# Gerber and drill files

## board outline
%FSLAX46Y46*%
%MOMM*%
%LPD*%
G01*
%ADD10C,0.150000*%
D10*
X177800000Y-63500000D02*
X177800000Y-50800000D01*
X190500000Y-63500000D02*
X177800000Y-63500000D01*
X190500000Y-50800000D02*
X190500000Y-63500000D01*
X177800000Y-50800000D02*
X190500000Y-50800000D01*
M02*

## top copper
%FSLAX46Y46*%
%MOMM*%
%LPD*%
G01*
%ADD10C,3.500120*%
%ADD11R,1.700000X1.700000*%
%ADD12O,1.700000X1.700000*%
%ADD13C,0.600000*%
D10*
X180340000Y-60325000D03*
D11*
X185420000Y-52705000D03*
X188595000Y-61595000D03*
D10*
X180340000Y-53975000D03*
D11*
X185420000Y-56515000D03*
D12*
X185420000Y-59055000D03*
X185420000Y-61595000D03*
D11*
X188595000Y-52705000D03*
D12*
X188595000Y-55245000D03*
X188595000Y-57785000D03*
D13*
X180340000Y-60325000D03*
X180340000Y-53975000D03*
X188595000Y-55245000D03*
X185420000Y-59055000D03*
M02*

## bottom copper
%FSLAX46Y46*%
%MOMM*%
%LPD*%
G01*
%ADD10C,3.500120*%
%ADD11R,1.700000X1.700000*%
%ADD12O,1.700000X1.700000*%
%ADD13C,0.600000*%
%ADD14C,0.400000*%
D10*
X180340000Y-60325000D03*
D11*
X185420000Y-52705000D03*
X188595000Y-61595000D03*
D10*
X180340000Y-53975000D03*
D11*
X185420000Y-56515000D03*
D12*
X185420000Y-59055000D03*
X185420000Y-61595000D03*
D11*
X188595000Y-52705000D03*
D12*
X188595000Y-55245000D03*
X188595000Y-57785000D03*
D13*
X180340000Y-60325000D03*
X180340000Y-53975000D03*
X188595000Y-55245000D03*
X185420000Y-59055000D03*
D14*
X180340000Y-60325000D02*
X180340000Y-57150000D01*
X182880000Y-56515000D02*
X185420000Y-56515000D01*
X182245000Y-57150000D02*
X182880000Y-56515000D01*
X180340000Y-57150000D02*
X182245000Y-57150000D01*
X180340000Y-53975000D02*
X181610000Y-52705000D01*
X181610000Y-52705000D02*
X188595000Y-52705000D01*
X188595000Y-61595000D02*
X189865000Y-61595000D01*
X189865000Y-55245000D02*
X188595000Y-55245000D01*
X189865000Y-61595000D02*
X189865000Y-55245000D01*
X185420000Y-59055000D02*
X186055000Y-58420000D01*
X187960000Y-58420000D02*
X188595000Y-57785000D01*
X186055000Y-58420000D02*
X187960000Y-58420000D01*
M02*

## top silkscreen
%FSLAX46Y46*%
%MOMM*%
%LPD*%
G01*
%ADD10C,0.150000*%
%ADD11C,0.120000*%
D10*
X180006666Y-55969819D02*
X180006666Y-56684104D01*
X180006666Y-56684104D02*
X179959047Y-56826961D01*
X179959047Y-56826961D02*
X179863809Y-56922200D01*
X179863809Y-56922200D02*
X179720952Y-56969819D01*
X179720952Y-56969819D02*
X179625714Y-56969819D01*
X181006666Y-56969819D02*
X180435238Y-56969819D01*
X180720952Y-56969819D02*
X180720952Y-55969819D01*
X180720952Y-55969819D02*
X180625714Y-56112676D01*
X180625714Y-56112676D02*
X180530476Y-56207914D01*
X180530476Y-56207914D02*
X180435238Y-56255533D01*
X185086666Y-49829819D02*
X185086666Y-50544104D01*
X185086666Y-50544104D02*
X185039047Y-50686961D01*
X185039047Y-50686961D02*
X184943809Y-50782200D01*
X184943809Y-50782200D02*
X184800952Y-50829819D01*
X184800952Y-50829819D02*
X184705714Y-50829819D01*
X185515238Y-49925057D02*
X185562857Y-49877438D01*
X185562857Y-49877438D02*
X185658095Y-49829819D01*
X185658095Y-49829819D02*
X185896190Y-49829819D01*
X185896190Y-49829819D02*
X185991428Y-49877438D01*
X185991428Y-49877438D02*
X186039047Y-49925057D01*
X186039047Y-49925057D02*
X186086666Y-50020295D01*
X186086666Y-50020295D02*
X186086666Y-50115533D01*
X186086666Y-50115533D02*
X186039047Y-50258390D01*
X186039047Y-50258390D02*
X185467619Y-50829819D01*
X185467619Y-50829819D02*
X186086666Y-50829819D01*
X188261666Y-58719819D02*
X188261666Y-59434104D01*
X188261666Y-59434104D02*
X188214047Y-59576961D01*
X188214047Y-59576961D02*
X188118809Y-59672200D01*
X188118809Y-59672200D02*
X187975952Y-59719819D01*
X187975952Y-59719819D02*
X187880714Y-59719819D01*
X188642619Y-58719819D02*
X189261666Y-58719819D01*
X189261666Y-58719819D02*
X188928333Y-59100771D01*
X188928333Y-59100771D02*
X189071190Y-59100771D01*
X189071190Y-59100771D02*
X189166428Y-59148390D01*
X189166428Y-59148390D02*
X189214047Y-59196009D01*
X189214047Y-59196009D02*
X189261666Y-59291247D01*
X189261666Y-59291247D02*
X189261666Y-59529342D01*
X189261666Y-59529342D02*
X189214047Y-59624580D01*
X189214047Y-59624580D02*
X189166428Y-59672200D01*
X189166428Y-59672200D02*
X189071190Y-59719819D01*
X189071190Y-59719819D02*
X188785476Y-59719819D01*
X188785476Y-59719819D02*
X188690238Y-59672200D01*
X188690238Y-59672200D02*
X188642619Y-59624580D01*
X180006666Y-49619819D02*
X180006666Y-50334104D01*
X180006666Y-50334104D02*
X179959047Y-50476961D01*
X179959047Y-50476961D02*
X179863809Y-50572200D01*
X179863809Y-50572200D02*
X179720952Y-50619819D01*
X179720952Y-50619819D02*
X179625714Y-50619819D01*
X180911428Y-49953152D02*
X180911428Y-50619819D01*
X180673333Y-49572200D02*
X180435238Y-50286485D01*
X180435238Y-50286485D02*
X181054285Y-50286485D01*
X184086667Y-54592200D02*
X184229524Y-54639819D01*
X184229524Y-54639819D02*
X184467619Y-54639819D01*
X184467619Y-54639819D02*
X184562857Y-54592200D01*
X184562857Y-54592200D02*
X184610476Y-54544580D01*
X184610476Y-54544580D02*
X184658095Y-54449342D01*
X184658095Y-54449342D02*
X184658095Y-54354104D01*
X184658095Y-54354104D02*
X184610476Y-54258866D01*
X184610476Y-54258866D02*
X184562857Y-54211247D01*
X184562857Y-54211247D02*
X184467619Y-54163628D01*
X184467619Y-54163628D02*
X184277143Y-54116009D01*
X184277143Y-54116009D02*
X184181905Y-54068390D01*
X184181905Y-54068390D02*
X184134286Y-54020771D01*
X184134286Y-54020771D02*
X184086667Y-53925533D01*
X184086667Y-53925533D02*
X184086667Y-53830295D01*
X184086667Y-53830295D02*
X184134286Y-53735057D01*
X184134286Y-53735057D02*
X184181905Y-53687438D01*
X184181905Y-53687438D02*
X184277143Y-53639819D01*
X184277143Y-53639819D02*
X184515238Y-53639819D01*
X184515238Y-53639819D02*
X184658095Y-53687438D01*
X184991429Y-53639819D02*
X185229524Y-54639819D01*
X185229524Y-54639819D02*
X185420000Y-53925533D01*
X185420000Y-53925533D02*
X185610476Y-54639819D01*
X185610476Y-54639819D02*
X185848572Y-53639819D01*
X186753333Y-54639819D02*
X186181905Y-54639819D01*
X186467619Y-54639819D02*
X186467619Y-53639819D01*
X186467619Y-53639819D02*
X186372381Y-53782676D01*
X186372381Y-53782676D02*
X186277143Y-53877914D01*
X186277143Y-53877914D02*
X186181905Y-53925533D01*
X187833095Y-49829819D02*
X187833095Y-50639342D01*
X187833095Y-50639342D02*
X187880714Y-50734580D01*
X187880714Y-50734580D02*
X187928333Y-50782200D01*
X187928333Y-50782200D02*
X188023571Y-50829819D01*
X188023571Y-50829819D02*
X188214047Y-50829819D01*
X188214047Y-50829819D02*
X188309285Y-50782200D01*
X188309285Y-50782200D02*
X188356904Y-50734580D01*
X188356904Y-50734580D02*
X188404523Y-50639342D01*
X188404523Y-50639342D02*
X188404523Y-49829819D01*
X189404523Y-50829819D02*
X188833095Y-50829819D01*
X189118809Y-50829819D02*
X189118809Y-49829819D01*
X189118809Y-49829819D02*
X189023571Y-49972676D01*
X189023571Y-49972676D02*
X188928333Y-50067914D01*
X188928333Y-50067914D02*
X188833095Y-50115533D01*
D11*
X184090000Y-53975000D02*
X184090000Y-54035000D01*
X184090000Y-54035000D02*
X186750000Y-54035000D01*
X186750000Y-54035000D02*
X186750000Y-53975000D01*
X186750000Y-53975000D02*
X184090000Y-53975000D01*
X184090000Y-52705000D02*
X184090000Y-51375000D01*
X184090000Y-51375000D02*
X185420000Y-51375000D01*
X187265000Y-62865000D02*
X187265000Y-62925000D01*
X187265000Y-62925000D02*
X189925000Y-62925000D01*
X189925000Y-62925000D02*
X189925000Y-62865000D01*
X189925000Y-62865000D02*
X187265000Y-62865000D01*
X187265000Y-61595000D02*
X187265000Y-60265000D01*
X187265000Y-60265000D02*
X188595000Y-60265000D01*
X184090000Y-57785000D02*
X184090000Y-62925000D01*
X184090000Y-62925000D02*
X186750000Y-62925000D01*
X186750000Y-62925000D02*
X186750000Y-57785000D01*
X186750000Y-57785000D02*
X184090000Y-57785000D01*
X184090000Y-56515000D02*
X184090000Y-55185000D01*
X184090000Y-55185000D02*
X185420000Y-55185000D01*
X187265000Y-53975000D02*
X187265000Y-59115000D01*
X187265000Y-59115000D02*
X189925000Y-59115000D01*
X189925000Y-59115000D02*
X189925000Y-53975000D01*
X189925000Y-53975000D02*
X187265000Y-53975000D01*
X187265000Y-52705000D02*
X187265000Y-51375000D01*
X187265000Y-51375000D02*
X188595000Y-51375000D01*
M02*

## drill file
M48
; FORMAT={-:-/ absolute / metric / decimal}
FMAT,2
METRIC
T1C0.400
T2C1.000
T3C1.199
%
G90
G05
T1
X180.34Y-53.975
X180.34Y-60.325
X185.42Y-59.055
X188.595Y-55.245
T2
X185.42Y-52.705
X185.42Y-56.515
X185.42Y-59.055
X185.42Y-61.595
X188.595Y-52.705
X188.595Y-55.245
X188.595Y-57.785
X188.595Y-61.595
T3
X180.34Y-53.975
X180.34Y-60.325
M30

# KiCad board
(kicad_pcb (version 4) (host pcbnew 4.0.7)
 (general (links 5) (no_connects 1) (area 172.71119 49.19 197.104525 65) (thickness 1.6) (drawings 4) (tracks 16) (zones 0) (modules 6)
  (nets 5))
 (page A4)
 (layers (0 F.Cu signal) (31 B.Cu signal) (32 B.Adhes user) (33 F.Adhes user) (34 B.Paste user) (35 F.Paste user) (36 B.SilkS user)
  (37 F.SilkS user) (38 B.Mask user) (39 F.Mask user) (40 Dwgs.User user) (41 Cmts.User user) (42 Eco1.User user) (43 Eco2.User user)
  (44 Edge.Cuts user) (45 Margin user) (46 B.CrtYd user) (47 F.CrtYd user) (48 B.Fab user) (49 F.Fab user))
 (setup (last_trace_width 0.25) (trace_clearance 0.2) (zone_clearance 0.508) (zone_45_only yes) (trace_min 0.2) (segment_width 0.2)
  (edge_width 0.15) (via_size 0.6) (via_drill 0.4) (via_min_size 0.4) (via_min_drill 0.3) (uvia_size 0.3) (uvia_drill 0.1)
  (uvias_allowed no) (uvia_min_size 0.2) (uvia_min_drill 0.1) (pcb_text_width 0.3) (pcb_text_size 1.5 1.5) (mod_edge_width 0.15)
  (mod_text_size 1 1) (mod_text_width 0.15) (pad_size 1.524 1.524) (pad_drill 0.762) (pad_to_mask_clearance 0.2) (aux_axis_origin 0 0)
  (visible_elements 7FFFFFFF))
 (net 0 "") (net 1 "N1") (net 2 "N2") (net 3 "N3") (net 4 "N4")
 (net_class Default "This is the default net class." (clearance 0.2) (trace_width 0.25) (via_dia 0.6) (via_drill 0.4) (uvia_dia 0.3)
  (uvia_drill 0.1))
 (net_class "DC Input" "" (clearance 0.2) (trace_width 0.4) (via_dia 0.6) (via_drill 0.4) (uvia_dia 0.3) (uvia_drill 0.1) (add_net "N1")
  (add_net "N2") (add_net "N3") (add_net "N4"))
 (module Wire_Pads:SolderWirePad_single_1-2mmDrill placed (layer F.Cu) (at 180.34 60.325)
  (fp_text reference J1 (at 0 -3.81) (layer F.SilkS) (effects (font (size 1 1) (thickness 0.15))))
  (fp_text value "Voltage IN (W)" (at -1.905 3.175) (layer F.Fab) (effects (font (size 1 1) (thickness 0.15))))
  (pad 1 thru_hole circle (at 0 0) (size 3.50012 3.50012) (drill 1.19888) (layers *.Cu *.Mask) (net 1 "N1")))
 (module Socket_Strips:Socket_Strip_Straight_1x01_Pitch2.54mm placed (layer F.Cu) (at 185.42 52.705)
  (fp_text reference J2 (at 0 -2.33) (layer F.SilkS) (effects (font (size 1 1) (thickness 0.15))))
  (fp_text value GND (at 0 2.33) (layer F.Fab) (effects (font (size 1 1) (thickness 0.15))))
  (fp_line (start -1.33 1.27) (end -1.33 1.33) (layer F.SilkS) (width 0.12))
  (fp_line (start -1.33 1.33) (end 1.33 1.33) (layer F.SilkS) (width 0.12))
  (fp_line (start 1.33 1.33) (end 1.33 1.27) (layer F.SilkS) (width 0.12))
  (fp_line (start 1.33 1.27) (end -1.33 1.27) (layer F.SilkS) (width 0.12))
  (fp_line (start -1.33 0) (end -1.33 -1.33) (layer F.SilkS) (width 0.12))
  (fp_line (start -1.33 -1.33) (end 0 -1.33) (layer F.SilkS) (width 0.12))
  (pad 1 thru_hole rect (at 0 0) (size 1.7 1.7) (drill 1) (layers *.Cu *.Mask) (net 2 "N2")))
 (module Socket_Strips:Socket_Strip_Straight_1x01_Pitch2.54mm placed (layer F.Cu) (at 188.595 61.595)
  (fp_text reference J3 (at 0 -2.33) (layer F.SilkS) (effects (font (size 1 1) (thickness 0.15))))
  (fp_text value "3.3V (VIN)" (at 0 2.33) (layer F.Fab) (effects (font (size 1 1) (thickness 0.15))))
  (fp_line (start -1.33 1.27) (end -1.33 1.33) (layer F.SilkS) (width 0.12))
  (fp_line (start -1.33 1.33) (end 1.33 1.33) (layer F.SilkS) (width 0.12))
  (fp_line (start 1.33 1.33) (end 1.33 1.27) (layer F.SilkS) (width 0.12))
  (fp_line (start 1.33 1.27) (end -1.33 1.27) (layer F.SilkS) (width 0.12))
  (fp_line (start -1.33 0) (end -1.33 -1.33) (layer F.SilkS) (width 0.12))
  (fp_line (start -1.33 -1.33) (end 0 -1.33) (layer F.SilkS) (width 0.12))
  (pad 1 thru_hole rect (at 0 0) (size 1.7 1.7) (drill 1) (layers *.Cu *.Mask) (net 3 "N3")))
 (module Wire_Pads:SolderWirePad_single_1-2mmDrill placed (layer F.Cu) (at 180.34 53.975)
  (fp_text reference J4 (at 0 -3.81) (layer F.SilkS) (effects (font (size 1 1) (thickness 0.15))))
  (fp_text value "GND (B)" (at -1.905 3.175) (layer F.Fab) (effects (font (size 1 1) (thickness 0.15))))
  (pad 1 thru_hole circle (at 0 0) (size 3.50012 3.50012) (drill 1.19888) (layers *.Cu *.Mask) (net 2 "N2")))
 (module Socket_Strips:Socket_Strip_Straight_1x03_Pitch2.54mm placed (layer F.Cu) (at 185.42 56.515)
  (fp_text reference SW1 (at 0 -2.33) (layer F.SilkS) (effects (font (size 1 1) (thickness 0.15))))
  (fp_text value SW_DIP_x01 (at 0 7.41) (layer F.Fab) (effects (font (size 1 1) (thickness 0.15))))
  (fp_line (start -1.33 1.27) (end -1.33 6.41) (layer F.SilkS) (width 0.12))
  (fp_line (start -1.33 6.41) (end 1.33 6.41) (layer F.SilkS) (width 0.12))
  (fp_line (start 1.33 6.41) (end 1.33 1.27) (layer F.SilkS) (width 0.12))
  (fp_line (start 1.33 1.27) (end -1.33 1.27) (layer F.SilkS) (width 0.12))
  (fp_line (start -1.33 0) (end -1.33 -1.33) (layer F.SilkS) (width 0.12))
  (fp_line (start -1.33 -1.33) (end 0 -1.33) (layer F.SilkS) (width 0.12))
  (pad 1 thru_hole rect (at 0 0) (size 1.7 1.7) (drill 1) (layers *.Cu *.Mask) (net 1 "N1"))
  (pad 2 thru_hole oval (at 0 2.54) (size 1.7 1.7) (drill 1) (layers *.Cu *.Mask) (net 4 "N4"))
  (pad 3 thru_hole oval (at 0 5.08) (size 1.7 1.7) (drill 1) (layers *.Cu *.Mask)))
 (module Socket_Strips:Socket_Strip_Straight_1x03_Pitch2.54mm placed (layer F.Cu) (at 188.595 52.705)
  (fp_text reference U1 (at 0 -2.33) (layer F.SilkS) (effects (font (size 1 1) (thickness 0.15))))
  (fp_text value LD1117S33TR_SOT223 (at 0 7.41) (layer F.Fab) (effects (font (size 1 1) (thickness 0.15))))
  (fp_line (start -1.33 1.27) (end -1.33 6.41) (layer F.SilkS) (width 0.12))
  (fp_line (start -1.33 6.41) (end 1.33 6.41) (layer F.SilkS) (width 0.12))
  (fp_line (start 1.33 6.41) (end 1.33 1.27) (layer F.SilkS) (width 0.12))
  (fp_line (start 1.33 1.27) (end -1.33 1.27) (layer F.SilkS) (width 0.12))
  (fp_line (start -1.33 0) (end -1.33 -1.33) (layer F.SilkS) (width 0.12))
  (fp_line (start -1.33 -1.33) (end 0 -1.33) (layer F.SilkS) (width 0.12))
  (pad 1 thru_hole rect (at 0 0) (size 1.7 1.7) (drill 1) (layers *.Cu *.Mask) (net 2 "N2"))
  (pad 2 thru_hole oval (at 0 2.54) (size 1.7 1.7) (drill 1) (layers *.Cu *.Mask) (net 3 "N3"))
  (pad 3 thru_hole oval (at 0 5.08) (size 1.7 1.7) (drill 1) (layers *.Cu *.Mask) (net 4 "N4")))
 (gr_line (start 177.8 63.5) (end 177.8 50.8) (angle 90) (layer Edge.Cuts) (width 0.15))
 (gr_line (start 190.5 63.5) (end 177.8 63.5) (angle 90) (layer Edge.Cuts) (width 0.15))
 (gr_line (start 190.5 50.8) (end 190.5 63.5) (angle 90) (layer Edge.Cuts) (width 0.15))
 (gr_line (start 177.8 50.8) (end 190.5 50.8) (angle 90) (layer Edge.Cuts) (width 0.15))
 (via (at 180.34 60.325) (size 0.6) (drill 0.4) (layers F.Cu B.Cu) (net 1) (status C00000))
 (segment (start 180.34 60.325) (end 180.34 57.15) (width 0.4) (layer B.Cu) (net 1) (status 400000))
 (segment (start 182.88 56.515) (end 185.42 56.515) (width 0.4) (layer B.Cu) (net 1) (status 800000))
 (segment (start 182.245 57.15) (end 182.88 56.515) (width 0.4) (layer B.Cu) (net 1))
 (segment (start 180.34 57.15) (end 182.245 57.15) (width 0.4) (layer B.Cu) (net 1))
 (segment (start 180.34 53.975) (end 181.61 52.705) (width 0.4) (layer B.Cu) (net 2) (status 400000))
 (segment (start 181.61 52.705) (end 188.595 52.705) (width 0.4) (layer B.Cu) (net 2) (status 800000))
 (via (at 180.34 53.975) (size 0.6) (drill 0.4) (layers F.Cu B.Cu) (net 2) (status C00000))
 (segment (start 188.595 61.595) (end 189.865 61.595) (width 0.4) (layer B.Cu) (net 3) (status 400000))
 (segment (start 189.865 55.245) (end 188.595 55.245) (width 0.4) (layer B.Cu) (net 3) (status 800000))
 (segment (start 189.865 61.595) (end 189.865 55.245) (width 0.4) (layer B.Cu) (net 3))
 (via (at 188.595 55.245) (size 0.6) (drill 0.4) (layers F.Cu B.Cu) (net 3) (status C00000))
 (via (at 185.42 59.055) (size 0.6) (drill 0.4) (layers F.Cu B.Cu) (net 4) (status C00000))
 (segment (start 185.42 59.055) (end 186.055 58.42) (width 0.4) (layer B.Cu) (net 4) (status 400000))
 (segment (start 187.96 58.42) (end 188.595 57.785) (width 0.4) (layer B.Cu) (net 4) (status 800000))
 (segment (start 186.055 58.42) (end 187.96 58.42) (width 0.4) (layer B.Cu) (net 4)))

